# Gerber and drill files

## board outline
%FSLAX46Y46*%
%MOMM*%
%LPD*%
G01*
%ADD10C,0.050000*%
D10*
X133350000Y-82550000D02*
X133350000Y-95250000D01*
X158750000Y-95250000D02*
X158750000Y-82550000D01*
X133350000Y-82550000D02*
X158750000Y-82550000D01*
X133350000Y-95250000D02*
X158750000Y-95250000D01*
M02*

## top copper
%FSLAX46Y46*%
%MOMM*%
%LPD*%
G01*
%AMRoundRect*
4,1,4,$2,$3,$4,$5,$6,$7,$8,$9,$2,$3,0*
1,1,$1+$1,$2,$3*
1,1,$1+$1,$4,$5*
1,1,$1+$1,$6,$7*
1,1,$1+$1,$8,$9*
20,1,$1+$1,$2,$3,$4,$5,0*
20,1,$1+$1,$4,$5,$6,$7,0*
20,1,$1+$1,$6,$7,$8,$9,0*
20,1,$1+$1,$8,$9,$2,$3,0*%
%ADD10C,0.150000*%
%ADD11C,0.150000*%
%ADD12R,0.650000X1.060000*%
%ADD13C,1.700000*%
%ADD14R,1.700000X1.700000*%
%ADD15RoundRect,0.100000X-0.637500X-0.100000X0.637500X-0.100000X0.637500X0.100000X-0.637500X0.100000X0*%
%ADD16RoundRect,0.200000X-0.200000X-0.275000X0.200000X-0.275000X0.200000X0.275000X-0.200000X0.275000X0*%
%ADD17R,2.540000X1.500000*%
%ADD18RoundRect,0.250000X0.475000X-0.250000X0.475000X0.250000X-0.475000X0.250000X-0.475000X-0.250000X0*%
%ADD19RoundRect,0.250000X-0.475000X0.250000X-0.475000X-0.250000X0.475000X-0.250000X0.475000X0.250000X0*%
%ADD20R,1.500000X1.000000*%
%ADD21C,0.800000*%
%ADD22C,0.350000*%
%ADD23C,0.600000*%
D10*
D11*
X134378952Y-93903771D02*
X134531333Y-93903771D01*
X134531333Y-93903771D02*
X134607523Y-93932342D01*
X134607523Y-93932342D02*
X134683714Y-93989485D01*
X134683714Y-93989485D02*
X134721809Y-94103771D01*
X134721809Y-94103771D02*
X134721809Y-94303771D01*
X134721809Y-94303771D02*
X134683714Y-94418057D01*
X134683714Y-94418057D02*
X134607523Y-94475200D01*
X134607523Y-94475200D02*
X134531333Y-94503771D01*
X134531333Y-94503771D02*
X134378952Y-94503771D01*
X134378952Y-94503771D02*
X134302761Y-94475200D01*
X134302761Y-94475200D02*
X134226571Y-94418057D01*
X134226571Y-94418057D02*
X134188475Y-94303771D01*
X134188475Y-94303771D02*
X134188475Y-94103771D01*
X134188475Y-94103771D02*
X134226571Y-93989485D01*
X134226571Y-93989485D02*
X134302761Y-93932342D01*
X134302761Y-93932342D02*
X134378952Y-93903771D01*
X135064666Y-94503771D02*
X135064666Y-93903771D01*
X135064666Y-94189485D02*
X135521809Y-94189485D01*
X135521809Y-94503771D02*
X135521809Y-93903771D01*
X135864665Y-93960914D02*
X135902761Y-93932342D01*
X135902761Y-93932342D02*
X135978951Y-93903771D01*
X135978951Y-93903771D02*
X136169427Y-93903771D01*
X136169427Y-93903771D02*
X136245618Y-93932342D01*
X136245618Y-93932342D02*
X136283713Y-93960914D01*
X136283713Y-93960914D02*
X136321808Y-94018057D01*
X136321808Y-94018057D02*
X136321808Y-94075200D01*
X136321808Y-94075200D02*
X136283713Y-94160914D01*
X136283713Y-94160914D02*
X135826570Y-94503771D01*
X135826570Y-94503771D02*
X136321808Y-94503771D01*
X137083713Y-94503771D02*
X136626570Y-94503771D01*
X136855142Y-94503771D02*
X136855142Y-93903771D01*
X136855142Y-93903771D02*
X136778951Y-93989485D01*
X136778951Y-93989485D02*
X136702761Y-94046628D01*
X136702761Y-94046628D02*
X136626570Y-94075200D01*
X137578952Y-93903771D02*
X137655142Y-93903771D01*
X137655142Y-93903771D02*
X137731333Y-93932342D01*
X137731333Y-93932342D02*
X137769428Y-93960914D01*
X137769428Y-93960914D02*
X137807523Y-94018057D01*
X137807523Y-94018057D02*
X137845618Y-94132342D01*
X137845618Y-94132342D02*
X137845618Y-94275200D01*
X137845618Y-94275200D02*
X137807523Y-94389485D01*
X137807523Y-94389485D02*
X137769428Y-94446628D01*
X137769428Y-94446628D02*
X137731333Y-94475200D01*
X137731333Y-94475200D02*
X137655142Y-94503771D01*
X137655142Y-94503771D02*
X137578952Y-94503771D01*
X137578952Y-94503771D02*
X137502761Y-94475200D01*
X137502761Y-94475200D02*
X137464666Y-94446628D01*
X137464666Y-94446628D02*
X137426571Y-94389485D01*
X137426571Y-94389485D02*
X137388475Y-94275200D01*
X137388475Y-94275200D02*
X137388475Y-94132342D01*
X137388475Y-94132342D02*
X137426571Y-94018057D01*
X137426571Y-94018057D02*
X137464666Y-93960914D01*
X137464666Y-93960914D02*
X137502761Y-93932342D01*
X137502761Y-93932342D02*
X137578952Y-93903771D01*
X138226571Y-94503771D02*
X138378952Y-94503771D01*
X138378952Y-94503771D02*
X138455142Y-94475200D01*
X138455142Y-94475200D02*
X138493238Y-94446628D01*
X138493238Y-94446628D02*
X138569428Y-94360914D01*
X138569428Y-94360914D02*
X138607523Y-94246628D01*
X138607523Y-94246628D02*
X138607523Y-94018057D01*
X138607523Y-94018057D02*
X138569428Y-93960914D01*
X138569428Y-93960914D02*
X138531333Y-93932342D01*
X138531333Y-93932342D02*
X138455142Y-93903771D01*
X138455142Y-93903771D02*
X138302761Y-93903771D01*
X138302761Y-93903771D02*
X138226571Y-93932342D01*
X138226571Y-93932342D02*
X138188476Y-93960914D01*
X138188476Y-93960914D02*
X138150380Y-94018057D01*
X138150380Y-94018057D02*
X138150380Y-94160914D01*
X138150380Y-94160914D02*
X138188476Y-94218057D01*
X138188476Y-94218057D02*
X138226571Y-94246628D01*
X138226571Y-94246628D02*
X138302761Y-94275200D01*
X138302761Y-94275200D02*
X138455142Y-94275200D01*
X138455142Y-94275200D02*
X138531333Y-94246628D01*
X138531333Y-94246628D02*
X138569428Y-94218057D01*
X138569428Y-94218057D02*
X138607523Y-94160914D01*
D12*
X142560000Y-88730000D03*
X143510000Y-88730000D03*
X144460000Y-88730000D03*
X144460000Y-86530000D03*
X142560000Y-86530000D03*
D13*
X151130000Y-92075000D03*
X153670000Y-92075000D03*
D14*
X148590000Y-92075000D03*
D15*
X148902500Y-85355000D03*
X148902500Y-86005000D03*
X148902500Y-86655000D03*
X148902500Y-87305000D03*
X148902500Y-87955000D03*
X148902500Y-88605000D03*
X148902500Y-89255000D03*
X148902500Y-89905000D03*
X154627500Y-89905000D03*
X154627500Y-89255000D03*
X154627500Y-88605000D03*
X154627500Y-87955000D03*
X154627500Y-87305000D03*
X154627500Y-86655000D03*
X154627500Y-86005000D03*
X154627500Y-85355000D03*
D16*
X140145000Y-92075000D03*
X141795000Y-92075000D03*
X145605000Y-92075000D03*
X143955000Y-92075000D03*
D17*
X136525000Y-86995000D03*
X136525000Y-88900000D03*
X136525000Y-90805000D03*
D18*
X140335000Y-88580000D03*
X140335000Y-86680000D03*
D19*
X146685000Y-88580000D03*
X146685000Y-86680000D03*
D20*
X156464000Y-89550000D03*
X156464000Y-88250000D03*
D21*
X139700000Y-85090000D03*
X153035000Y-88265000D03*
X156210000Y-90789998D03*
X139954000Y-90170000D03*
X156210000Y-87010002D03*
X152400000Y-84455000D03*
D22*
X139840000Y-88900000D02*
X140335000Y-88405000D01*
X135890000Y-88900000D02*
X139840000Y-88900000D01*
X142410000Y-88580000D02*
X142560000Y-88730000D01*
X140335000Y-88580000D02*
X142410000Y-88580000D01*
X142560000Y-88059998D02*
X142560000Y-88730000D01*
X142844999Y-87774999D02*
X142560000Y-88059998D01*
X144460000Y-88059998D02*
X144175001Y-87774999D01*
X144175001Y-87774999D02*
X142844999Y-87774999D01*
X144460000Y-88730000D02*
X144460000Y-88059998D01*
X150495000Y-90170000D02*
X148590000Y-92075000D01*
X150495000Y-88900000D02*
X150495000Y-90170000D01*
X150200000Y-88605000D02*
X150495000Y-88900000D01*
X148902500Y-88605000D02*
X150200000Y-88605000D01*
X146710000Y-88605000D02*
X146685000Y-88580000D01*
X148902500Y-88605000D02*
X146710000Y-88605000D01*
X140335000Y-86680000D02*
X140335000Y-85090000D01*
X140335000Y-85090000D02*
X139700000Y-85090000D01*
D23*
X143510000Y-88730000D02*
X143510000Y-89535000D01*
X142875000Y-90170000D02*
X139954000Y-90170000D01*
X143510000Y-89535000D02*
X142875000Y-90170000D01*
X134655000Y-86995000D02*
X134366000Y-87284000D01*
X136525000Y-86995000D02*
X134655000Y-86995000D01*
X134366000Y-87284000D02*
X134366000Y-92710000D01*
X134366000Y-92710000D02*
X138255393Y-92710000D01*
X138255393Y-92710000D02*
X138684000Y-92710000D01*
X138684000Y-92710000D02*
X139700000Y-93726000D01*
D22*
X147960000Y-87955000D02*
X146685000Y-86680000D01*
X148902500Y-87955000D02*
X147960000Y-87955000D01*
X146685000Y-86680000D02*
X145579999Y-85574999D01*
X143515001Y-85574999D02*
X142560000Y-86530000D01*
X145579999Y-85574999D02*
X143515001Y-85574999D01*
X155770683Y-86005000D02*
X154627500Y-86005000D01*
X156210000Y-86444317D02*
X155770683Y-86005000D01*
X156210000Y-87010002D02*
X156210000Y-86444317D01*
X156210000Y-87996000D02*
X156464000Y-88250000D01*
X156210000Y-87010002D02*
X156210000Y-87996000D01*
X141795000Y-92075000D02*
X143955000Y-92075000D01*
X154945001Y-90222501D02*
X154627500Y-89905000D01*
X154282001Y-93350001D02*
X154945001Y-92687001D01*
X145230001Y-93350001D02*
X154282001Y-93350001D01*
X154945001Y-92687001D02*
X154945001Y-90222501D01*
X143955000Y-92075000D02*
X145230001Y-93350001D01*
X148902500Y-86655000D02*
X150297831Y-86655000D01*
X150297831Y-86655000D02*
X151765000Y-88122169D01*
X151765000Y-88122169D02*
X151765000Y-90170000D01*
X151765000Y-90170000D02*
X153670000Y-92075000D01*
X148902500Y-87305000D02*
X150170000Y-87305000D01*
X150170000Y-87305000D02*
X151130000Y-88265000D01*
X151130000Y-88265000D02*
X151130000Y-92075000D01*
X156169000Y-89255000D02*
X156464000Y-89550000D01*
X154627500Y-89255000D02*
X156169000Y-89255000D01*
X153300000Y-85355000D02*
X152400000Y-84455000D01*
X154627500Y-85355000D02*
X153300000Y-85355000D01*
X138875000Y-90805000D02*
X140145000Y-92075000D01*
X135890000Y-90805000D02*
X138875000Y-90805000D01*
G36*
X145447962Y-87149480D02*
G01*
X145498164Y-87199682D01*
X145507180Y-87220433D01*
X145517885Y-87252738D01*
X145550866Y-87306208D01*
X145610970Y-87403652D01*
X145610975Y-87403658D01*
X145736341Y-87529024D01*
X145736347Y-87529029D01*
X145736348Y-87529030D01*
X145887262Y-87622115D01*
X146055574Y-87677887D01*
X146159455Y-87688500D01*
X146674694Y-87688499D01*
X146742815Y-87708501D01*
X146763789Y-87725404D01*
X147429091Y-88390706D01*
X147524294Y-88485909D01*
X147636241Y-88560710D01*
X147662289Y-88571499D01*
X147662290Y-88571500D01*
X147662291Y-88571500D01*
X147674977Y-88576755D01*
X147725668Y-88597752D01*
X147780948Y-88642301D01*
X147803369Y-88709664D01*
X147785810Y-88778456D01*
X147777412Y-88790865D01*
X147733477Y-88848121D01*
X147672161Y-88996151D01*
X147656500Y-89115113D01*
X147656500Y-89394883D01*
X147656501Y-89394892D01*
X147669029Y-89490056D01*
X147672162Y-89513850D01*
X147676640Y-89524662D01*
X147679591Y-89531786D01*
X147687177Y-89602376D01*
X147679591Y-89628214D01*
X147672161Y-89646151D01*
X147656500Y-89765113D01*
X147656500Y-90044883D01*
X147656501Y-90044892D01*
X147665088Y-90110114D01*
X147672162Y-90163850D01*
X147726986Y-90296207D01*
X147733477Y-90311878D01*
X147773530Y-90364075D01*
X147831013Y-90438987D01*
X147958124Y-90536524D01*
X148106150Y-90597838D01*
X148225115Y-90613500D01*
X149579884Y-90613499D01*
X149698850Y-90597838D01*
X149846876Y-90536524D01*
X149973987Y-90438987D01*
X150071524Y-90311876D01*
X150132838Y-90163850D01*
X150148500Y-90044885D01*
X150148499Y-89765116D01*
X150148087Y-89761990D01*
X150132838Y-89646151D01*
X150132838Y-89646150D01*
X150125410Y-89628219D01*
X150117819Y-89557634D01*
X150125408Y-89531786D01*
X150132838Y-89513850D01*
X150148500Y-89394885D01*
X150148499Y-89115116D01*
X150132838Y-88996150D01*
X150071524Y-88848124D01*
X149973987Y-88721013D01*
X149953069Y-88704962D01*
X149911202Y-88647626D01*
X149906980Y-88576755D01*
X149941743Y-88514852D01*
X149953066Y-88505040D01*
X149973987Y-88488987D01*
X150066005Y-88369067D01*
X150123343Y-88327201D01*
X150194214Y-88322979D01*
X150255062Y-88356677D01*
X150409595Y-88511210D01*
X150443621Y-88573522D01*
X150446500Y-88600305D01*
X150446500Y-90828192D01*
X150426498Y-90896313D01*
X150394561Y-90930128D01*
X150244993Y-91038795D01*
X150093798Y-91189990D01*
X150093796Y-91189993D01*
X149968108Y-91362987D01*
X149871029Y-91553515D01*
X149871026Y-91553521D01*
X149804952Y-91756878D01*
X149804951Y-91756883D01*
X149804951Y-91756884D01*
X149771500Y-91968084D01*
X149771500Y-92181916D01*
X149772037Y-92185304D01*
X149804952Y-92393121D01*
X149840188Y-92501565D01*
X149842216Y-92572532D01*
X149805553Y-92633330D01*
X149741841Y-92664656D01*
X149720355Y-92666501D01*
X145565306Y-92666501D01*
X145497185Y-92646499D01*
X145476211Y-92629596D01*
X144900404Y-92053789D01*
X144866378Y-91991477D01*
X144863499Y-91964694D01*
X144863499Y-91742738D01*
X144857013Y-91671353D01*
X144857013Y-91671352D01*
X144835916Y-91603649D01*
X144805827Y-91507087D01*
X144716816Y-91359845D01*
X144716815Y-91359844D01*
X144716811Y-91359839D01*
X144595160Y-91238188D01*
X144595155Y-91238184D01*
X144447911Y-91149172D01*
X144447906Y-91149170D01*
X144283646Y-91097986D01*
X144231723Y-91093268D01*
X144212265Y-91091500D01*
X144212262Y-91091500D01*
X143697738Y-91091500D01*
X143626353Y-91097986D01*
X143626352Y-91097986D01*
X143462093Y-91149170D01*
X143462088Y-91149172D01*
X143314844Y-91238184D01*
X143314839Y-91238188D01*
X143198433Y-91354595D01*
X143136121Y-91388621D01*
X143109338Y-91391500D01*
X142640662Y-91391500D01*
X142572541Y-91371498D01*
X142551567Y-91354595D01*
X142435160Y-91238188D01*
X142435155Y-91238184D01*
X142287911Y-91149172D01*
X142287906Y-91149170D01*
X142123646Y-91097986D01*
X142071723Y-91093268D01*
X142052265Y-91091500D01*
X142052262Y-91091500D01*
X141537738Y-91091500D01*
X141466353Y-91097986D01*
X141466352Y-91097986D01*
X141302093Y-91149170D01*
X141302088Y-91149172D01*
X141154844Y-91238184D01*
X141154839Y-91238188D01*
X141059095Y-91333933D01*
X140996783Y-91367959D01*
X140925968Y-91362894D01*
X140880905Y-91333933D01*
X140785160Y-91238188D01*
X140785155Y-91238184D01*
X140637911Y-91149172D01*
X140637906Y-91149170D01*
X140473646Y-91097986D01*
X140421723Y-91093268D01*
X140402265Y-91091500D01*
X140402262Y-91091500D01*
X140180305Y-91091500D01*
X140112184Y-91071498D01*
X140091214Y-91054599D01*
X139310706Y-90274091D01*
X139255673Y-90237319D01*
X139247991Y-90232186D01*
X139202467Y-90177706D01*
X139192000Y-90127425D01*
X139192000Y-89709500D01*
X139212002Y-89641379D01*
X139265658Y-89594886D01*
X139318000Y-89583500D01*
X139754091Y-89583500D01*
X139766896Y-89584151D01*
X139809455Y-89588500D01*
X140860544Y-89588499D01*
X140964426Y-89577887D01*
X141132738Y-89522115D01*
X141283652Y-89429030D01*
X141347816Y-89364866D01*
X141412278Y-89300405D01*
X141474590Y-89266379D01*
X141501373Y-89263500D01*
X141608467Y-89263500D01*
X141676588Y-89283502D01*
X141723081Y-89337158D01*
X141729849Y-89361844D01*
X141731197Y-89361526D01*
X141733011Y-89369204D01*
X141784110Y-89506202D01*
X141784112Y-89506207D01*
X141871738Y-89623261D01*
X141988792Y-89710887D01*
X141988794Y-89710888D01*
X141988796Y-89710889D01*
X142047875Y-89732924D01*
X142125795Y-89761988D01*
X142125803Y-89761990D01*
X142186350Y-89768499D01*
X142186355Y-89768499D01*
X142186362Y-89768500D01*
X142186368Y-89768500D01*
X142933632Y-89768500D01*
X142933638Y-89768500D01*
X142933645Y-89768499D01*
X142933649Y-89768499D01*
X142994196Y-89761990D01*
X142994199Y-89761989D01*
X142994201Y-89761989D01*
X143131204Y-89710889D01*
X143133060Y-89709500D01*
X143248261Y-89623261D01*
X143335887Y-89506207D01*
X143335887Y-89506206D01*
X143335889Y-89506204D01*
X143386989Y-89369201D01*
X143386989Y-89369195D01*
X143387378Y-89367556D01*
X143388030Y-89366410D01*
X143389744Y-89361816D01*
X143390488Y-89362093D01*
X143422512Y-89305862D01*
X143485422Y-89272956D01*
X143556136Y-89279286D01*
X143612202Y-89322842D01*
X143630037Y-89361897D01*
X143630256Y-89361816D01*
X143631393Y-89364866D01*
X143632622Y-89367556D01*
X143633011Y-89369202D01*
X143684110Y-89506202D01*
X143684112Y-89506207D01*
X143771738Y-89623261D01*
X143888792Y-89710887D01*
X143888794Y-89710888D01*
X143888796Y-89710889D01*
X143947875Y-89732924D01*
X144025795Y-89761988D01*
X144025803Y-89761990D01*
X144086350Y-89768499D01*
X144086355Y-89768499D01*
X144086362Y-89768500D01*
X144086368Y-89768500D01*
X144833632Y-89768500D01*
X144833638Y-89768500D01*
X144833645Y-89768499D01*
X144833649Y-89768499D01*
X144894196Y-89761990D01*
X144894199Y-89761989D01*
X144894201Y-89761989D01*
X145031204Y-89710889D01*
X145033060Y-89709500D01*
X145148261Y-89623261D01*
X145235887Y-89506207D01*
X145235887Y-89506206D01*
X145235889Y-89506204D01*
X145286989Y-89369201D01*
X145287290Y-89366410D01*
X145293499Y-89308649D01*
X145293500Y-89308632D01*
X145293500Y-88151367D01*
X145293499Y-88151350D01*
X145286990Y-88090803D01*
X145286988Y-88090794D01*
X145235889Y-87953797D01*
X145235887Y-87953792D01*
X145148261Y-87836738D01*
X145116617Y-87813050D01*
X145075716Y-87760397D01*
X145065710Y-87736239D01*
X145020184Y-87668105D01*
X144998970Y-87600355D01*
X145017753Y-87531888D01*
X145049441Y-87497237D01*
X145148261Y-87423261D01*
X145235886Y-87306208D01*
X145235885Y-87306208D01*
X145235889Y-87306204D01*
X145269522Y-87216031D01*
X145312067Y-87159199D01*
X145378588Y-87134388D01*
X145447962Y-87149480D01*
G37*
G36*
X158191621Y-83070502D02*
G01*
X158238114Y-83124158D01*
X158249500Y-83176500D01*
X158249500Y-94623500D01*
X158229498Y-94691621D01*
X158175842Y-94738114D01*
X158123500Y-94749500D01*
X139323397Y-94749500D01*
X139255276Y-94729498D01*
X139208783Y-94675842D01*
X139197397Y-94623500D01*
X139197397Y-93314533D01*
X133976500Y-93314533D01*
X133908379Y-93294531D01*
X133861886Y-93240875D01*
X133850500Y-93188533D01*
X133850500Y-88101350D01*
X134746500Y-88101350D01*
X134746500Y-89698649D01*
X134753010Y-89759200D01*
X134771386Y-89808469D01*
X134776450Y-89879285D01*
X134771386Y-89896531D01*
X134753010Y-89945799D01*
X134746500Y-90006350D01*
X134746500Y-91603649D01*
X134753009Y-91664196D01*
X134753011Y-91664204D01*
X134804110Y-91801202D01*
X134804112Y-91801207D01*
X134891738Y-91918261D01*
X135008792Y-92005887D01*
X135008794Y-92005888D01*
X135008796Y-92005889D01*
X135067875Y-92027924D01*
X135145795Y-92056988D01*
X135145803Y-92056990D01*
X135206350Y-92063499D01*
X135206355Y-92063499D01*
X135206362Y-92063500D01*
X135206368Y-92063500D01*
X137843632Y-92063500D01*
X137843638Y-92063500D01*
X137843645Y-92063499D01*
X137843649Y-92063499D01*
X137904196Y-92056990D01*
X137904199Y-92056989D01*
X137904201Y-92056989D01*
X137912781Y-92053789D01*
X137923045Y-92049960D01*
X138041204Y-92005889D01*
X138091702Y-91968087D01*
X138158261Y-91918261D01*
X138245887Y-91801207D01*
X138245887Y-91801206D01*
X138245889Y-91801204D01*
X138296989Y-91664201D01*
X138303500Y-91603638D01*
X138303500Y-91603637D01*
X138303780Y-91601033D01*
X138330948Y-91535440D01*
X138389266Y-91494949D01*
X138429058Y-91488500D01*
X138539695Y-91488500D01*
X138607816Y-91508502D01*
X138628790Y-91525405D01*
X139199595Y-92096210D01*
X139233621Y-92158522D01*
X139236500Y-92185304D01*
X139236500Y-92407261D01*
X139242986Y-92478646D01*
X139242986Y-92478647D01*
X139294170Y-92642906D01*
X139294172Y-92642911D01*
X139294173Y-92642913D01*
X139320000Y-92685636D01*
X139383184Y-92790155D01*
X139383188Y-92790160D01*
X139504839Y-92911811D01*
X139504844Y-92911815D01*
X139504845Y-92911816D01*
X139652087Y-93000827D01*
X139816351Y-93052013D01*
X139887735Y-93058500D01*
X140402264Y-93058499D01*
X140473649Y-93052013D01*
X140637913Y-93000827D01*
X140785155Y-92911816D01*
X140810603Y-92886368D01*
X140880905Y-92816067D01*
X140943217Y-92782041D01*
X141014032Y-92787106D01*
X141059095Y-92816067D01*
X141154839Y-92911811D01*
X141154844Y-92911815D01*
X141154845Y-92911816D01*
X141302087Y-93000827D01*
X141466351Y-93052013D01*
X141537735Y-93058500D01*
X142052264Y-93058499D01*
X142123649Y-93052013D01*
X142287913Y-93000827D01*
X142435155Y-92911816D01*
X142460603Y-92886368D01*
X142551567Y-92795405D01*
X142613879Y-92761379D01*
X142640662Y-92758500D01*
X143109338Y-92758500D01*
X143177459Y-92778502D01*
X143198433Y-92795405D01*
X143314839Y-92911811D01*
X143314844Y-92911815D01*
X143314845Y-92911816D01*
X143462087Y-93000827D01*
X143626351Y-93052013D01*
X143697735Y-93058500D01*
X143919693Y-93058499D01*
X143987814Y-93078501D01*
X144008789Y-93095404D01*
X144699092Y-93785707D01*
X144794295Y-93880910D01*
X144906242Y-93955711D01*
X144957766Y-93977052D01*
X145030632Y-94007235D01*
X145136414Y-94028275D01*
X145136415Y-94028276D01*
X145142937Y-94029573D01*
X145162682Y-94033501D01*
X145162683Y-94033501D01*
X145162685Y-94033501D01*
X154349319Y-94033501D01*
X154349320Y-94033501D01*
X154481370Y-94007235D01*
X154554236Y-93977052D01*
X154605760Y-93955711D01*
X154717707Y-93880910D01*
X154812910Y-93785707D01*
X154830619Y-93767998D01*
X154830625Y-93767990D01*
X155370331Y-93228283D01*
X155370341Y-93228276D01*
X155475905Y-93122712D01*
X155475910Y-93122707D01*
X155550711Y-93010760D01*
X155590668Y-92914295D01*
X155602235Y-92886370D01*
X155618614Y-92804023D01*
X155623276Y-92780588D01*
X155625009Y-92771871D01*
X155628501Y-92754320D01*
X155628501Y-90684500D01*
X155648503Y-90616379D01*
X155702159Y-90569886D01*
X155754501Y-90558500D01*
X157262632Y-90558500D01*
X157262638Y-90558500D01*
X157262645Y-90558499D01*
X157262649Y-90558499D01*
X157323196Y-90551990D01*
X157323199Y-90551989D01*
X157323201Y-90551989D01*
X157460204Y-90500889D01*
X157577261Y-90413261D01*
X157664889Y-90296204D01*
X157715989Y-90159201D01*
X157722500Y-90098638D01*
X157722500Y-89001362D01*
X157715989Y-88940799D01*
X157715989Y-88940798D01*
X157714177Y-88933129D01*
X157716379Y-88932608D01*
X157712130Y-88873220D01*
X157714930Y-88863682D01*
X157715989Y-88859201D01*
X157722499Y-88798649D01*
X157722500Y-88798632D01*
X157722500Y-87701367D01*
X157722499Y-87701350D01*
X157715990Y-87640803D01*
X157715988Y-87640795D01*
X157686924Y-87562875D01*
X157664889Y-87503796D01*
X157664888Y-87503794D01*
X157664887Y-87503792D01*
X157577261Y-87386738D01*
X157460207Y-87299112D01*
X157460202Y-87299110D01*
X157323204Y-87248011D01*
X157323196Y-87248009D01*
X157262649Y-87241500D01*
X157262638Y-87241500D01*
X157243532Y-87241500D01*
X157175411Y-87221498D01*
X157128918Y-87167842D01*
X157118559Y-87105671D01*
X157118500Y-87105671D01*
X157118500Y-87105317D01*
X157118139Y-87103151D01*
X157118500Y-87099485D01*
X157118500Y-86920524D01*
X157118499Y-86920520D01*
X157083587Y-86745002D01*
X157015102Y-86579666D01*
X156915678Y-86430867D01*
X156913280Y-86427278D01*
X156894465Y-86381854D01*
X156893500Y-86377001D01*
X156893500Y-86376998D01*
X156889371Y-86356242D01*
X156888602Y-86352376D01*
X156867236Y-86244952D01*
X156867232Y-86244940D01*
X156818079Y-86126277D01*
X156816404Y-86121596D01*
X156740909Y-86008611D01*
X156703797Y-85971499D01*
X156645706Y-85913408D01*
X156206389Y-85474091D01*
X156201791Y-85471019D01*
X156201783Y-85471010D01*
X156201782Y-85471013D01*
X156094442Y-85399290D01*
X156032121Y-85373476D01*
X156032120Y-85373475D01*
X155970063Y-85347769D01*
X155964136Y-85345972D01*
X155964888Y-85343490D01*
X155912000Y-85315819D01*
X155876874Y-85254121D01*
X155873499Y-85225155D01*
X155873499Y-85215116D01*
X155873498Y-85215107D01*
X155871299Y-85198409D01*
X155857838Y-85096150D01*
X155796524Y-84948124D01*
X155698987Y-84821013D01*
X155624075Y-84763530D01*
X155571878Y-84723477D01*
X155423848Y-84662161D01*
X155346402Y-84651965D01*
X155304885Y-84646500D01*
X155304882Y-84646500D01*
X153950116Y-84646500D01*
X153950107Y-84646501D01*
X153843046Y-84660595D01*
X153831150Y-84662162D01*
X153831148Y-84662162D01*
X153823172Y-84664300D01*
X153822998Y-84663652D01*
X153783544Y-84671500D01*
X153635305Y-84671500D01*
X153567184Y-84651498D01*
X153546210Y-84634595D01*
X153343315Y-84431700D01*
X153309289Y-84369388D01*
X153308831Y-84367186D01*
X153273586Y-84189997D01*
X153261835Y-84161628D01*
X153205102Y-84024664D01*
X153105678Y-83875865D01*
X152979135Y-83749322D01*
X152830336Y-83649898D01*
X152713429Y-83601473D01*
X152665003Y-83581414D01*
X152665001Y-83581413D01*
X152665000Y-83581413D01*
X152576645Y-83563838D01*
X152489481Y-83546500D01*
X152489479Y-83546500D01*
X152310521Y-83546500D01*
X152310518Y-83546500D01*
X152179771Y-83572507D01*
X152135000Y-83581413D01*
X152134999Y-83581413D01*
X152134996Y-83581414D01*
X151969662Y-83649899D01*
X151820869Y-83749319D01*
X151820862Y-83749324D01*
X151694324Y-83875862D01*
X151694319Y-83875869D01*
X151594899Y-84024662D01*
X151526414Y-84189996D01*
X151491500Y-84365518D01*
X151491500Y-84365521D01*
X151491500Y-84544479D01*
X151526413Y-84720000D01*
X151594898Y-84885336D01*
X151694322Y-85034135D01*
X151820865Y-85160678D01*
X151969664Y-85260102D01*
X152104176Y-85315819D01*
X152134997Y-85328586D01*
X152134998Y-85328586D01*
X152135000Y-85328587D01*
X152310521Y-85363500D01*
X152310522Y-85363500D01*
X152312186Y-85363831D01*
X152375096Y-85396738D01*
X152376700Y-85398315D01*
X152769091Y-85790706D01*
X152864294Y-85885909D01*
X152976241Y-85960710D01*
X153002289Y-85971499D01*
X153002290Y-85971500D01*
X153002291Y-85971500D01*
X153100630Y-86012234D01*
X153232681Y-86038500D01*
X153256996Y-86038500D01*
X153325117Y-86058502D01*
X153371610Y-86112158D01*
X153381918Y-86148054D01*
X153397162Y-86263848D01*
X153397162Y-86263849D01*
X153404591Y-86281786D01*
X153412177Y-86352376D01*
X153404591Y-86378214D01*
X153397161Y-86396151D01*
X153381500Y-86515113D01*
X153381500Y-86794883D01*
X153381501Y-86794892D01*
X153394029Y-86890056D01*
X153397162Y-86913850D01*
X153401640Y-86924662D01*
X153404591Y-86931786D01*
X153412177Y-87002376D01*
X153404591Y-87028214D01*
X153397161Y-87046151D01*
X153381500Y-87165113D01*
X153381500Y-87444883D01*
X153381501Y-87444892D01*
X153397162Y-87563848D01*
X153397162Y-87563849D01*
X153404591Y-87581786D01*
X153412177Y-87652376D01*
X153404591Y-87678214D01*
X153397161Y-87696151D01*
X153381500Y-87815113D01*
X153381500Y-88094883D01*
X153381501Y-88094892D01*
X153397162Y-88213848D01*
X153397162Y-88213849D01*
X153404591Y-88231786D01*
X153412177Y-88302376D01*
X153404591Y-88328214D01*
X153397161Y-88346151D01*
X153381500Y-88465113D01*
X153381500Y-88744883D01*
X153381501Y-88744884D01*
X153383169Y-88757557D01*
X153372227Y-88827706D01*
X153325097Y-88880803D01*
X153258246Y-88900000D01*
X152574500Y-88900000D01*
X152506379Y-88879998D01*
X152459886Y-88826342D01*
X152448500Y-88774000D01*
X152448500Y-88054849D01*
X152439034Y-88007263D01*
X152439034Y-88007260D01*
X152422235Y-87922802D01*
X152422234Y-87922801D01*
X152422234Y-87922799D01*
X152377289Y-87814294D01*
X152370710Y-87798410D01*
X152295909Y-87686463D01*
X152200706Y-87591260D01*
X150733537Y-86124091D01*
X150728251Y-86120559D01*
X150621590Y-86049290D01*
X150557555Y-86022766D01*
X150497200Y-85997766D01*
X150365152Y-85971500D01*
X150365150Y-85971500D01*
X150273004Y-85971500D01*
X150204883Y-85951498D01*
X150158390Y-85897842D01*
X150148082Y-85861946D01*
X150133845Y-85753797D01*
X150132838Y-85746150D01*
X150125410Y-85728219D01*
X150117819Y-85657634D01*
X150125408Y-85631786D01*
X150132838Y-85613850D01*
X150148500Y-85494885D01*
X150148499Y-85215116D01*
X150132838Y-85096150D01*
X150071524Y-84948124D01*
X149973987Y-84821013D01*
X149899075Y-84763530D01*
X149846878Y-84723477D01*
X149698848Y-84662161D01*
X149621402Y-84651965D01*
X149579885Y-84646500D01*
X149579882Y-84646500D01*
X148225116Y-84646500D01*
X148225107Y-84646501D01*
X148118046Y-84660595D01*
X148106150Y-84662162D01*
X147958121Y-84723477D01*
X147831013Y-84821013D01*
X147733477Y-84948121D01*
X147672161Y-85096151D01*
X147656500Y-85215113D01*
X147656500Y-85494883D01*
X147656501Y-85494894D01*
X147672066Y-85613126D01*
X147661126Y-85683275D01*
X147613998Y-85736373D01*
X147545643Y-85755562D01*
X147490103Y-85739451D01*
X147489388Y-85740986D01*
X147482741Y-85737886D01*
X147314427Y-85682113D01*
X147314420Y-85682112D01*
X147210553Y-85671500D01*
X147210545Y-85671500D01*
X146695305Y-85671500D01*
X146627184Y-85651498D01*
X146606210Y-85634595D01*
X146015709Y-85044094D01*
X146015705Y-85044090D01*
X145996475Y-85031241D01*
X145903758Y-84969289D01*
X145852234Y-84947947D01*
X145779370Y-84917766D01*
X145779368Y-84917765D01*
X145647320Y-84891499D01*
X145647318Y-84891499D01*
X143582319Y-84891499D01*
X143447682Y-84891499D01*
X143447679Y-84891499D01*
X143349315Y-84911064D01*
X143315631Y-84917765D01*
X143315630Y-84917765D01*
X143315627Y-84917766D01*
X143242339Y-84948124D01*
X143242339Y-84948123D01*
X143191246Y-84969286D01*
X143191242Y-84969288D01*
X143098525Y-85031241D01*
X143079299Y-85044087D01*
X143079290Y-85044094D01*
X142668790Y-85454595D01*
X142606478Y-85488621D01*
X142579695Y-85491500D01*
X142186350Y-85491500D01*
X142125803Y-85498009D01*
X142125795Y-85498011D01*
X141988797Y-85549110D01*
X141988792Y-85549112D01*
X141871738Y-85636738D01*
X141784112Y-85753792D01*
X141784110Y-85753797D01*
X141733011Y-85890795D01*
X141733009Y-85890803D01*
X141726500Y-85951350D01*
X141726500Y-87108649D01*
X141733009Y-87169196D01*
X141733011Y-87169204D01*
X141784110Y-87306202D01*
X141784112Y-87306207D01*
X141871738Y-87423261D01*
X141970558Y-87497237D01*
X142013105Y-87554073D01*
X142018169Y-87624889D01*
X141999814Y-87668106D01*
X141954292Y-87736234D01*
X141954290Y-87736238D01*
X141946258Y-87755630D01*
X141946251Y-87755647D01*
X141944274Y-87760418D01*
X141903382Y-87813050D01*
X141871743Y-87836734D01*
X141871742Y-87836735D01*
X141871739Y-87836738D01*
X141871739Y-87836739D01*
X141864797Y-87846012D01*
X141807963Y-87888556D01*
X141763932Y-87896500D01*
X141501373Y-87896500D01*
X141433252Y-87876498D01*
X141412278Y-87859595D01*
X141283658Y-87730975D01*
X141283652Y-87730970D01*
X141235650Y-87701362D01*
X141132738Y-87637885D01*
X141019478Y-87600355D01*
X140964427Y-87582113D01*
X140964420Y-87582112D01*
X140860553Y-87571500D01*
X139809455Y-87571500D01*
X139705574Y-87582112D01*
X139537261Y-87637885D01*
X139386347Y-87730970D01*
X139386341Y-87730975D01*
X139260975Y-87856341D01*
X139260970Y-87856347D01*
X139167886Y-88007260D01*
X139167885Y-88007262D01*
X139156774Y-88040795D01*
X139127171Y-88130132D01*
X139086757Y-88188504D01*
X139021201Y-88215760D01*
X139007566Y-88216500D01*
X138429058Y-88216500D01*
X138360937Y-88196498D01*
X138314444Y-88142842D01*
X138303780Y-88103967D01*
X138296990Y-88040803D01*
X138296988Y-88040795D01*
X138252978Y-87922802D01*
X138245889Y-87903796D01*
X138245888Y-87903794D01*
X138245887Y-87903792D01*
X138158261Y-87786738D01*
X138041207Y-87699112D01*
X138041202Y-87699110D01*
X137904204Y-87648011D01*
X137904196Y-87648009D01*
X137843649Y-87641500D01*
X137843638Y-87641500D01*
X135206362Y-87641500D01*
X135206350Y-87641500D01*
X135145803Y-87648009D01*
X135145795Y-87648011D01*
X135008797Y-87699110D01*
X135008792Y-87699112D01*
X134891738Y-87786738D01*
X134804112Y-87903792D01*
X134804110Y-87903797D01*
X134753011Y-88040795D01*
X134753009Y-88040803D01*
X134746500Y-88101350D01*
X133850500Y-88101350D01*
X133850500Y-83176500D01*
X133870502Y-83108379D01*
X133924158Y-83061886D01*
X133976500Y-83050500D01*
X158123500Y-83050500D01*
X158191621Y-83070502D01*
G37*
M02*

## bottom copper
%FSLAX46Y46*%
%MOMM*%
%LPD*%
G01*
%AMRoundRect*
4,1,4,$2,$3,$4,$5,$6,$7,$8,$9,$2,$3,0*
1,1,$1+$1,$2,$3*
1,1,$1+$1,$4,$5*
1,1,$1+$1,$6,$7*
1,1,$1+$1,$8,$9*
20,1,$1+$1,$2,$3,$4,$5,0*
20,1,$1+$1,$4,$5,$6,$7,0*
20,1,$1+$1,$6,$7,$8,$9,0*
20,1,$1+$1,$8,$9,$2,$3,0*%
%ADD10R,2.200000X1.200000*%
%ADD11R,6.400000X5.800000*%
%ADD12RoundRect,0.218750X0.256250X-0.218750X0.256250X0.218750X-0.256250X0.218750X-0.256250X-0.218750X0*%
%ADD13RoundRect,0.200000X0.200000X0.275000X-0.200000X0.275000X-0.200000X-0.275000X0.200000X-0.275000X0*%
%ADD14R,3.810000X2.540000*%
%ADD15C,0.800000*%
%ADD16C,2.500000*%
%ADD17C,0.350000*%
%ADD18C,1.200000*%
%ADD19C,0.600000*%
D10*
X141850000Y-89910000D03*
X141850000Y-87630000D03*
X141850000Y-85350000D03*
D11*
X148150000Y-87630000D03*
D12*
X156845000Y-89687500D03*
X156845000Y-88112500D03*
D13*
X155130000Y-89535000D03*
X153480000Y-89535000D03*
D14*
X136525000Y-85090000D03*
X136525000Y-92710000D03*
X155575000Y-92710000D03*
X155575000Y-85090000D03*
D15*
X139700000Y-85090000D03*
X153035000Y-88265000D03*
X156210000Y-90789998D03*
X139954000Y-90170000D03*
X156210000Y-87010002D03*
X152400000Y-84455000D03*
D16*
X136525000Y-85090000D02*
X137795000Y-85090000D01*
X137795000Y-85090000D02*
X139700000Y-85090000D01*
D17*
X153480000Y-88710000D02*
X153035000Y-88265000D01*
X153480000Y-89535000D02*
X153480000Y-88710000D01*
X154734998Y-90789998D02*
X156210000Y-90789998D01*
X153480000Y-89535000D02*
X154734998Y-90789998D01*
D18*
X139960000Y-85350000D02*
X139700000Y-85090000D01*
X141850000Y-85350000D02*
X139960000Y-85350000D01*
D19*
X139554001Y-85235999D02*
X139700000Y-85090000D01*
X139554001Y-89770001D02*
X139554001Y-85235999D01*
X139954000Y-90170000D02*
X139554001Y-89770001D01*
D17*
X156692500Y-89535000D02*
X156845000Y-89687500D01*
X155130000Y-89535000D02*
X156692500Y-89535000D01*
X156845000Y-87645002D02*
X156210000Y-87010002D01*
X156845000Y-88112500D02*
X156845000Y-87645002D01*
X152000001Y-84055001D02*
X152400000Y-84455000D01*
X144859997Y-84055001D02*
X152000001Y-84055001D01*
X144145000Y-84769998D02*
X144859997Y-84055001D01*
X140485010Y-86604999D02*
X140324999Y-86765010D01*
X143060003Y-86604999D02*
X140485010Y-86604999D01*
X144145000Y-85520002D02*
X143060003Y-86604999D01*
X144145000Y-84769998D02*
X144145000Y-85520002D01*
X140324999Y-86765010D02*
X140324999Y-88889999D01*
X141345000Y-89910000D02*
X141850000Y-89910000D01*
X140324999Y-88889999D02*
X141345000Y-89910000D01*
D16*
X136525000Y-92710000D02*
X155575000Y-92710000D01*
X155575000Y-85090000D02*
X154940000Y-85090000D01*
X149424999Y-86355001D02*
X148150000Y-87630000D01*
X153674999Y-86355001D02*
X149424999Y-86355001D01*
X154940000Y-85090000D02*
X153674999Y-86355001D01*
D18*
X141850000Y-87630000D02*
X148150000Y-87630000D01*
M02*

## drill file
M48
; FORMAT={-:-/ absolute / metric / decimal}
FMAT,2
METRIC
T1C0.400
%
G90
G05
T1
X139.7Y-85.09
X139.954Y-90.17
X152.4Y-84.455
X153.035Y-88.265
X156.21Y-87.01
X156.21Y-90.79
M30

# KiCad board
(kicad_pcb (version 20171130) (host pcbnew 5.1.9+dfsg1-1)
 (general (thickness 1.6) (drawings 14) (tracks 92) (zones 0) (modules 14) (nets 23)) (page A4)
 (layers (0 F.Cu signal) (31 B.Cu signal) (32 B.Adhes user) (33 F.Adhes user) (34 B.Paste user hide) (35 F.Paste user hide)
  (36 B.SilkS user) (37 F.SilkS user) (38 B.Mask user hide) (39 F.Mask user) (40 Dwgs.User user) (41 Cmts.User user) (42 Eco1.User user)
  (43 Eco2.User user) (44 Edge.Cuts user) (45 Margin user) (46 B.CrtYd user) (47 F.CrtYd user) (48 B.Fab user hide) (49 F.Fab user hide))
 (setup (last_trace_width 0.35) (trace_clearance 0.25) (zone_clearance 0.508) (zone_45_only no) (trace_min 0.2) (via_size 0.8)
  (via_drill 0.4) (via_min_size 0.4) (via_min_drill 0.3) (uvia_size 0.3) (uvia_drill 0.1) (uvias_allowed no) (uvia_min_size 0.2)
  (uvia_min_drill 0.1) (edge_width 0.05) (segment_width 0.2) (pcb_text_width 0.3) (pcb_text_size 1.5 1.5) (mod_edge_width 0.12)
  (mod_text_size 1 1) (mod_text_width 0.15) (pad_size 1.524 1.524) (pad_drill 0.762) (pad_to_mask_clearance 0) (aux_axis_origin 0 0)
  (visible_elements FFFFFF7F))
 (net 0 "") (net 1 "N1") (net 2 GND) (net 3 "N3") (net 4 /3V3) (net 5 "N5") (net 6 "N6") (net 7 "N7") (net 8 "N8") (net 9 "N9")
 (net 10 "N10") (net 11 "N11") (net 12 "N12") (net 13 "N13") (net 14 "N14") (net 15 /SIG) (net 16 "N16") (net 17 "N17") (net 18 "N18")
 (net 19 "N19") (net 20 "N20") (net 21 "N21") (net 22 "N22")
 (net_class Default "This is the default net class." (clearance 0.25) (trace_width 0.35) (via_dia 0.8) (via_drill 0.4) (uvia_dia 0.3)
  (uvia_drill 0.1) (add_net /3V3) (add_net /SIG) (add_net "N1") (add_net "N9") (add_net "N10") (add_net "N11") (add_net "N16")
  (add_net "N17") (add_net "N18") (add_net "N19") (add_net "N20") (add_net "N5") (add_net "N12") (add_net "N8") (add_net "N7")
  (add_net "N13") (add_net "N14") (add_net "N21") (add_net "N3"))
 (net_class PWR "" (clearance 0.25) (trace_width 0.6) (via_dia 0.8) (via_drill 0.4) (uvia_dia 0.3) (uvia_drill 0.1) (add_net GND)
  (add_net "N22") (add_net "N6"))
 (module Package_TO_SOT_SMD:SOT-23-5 (layer F.Cu) (at 143.51 87.63 90)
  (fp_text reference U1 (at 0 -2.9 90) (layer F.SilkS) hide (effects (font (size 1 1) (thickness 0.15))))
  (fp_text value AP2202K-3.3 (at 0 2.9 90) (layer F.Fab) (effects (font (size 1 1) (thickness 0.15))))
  (pad 1 smd rect (at -1.1 -0.95 90) (size 1.06 0.65) (layers F.Cu F.Paste F.Mask) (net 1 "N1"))
  (pad 2 smd rect (at -1.1 0 90) (size 1.06 0.65) (layers F.Cu F.Paste F.Mask) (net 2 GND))
  (pad 3 smd rect (at -1.1 0.95 90) (size 1.06 0.65) (layers F.Cu F.Paste F.Mask) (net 1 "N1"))
  (pad 4 smd rect (at 1.1 0.95 90) (size 1.06 0.65) (layers F.Cu F.Paste F.Mask) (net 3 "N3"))
  (pad 5 smd rect (at 1.1 -0.95 90) (size 1.06 0.65) (layers F.Cu F.Paste F.Mask) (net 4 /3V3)))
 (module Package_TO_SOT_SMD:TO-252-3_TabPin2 (layer B.Cu) (at 146.05 87.63)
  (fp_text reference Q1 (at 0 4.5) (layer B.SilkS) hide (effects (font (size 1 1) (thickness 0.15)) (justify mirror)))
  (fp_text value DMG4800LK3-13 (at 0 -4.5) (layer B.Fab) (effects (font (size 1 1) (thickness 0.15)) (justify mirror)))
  (pad 1 smd rect (at -4.2 2.28) (size 2.2 1.2) (layers B.Cu B.Paste B.Mask) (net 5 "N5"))
  (pad 2 smd rect (at -4.2 0) (size 2.2 1.2) (layers B.Cu B.Paste B.Mask) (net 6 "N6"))
  (pad 3 smd rect (at -4.2 -2.28) (size 2.2 1.2) (layers B.Cu B.Paste B.Mask) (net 2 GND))
  (pad 2 smd rect (at 2.1 0) (size 6.4 5.8) (layers B.Cu B.Mask) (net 6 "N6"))
  (pad "" smd rect (at 3.775 -1.525) (size 3.05 2.75) (layers B.Paste))
  (pad "" smd rect (at 0.425 1.525) (size 3.05 2.75) (layers B.Paste))
  (pad "" smd rect (at 3.775 1.525) (size 3.05 2.75) (layers B.Paste))
  (pad "" smd rect (at 0.425 -1.525) (size 3.05 2.75) (layers B.Paste)))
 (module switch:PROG (layer F.Cu) (at 151.13 92.075 90)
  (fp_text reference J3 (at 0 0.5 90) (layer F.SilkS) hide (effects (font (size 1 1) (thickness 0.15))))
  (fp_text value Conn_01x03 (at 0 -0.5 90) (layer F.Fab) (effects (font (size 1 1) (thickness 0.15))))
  (pad 2 smd circle (at 0 0 90) (size 1.7 1.7) (layers F.Cu F.Paste F.Mask) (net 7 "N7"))
  (pad 3 smd circle (at 0 2.54 90) (size 1.7 1.7) (layers F.Cu F.Paste F.Mask) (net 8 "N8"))
  (pad 1 smd rect (at 0 -2.54 90) (size 1.7 1.7) (layers F.Cu F.Paste F.Mask) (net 2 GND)))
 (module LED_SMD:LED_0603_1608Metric (layer B.Cu) (at 156.845 88.9 90)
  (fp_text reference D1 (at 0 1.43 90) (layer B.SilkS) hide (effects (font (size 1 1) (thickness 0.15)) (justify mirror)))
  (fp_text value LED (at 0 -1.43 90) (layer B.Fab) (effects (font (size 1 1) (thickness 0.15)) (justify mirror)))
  (pad 1 smd roundrect (at -0.7875 0 90) (size 0.875 0.95) (layers B.Cu B.Paste B.Mask) (roundrect_rratio 0.25) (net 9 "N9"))
  (pad 2 smd roundrect (at 0.7875 0 90) (size 0.875 0.95) (layers B.Cu B.Paste B.Mask) (roundrect_rratio 0.25) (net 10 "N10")))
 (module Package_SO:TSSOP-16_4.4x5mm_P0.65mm (layer F.Cu) (at 151.765 87.63)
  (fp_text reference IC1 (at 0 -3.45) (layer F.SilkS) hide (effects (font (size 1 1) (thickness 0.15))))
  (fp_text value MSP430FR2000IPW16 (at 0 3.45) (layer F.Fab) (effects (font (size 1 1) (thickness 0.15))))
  (pad 1 smd roundrect (at -2.8625 -2.275) (size 1.475 0.4) (layers F.Cu F.Paste F.Mask) (roundrect_rratio 0.25) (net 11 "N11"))
  (pad 2 smd roundrect (at -2.8625 -1.625) (size 1.475 0.4) (layers F.Cu F.Paste F.Mask) (roundrect_rratio 0.25) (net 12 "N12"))
  (pad 3 smd roundrect (at -2.8625 -0.975) (size 1.475 0.4) (layers F.Cu F.Paste F.Mask) (roundrect_rratio 0.25) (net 8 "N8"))
  (pad 4 smd roundrect (at -2.8625 -0.325) (size 1.475 0.4) (layers F.Cu F.Paste F.Mask) (roundrect_rratio 0.25) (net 7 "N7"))
  (pad 5 smd roundrect (at -2.8625 0.325) (size 1.475 0.4) (layers F.Cu F.Paste F.Mask) (roundrect_rratio 0.25) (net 4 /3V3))
  (pad 6 smd roundrect (at -2.8625 0.975) (size 1.475 0.4) (layers F.Cu F.Paste F.Mask) (roundrect_rratio 0.25) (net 2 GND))
  (pad 7 smd roundrect (at -2.8625 1.625) (size 1.475 0.4) (layers F.Cu F.Paste F.Mask) (roundrect_rratio 0.25) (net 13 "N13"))
  (pad 8 smd roundrect (at -2.8625 2.275) (size 1.475 0.4) (layers F.Cu F.Paste F.Mask) (roundrect_rratio 0.25) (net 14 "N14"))
  (pad 9 smd roundrect (at 2.8625 2.275) (size 1.475 0.4) (layers F.Cu F.Paste F.Mask) (roundrect_rratio 0.25) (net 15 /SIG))
  (pad 10 smd roundrect (at 2.8625 1.625) (size 1.475 0.4) (layers F.Cu F.Paste F.Mask) (roundrect_rratio 0.25) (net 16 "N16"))
  (pad 11 smd roundrect (at 2.8625 0.975) (size 1.475 0.4) (layers F.Cu F.Paste F.Mask) (roundrect_rratio 0.25) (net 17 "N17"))
  (pad 12 smd roundrect (at 2.8625 0.325) (size 1.475 0.4) (layers F.Cu F.Paste F.Mask) (roundrect_rratio 0.25) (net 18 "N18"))
  (pad 13 smd roundrect (at 2.8625 -0.325) (size 1.475 0.4) (layers F.Cu F.Paste F.Mask) (roundrect_rratio 0.25) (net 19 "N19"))
  (pad 14 smd roundrect (at 2.8625 -0.975) (size 1.475 0.4) (layers F.Cu F.Paste F.Mask) (roundrect_rratio 0.25) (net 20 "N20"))
  (pad 15 smd roundrect (at 2.8625 -1.625) (size 1.475 0.4) (layers F.Cu F.Paste F.Mask) (roundrect_rratio 0.25) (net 10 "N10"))
  (pad 16 smd roundrect (at 2.8625 -2.275) (size 1.475 0.4) (layers F.Cu F.Paste F.Mask) (roundrect_rratio 0.25) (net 5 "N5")))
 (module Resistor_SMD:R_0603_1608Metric (layer F.Cu) (at 140.97 92.075)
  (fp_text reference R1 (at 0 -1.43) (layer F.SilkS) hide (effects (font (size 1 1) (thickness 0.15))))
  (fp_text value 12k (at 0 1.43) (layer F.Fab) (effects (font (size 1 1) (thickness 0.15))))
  (pad 1 smd roundrect (at -0.825 0) (size 0.8 0.95) (layers F.Cu F.Paste F.Mask) (roundrect_rratio 0.25) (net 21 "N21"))
  (pad 2 smd roundrect (at 0.825 0) (size 0.8 0.95) (layers F.Cu F.Paste F.Mask) (roundrect_rratio 0.25) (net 15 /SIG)))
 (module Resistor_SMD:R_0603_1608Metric (layer F.Cu) (at 144.78 92.075)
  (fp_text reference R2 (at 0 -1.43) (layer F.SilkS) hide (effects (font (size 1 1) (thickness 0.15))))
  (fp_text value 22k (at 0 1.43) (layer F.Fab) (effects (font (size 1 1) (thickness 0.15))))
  (pad 2 smd roundrect (at 0.825 0) (size 0.8 0.95) (layers F.Cu F.Paste F.Mask) (roundrect_rratio 0.25) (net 2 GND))
  (pad 1 smd roundrect (at -0.825 0) (size 0.8 0.95) (layers F.Cu F.Paste F.Mask) (roundrect_rratio 0.25) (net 15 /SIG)))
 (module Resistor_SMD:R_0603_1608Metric (layer B.Cu) (at 154.305 89.535 180)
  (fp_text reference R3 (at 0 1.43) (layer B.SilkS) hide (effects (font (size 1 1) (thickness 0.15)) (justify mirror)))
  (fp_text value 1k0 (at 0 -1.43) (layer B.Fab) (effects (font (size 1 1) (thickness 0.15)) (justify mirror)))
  (pad 1 smd roundrect (at -0.825 0 180) (size 0.8 0.95) (layers B.Cu B.Paste B.Mask) (roundrect_rratio 0.25) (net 9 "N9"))
  (pad 2 smd roundrect (at 0.825 0 180) (size 0.8 0.95) (layers B.Cu B.Paste B.Mask) (roundrect_rratio 0.25) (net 2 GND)))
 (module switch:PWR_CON (layer B.Cu) (at 136.525 88.9 180)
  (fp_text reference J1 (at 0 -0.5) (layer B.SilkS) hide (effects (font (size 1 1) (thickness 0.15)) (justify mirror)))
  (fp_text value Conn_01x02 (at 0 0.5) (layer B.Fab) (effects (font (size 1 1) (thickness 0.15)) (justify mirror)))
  (pad 1 smd rect (at 0 3.81 180) (size 3.81 2.54) (layers B.Cu B.Paste B.Mask) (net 2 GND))
  (pad 2 smd rect (at 0 -3.81 180) (size 3.81 2.54) (layers B.Cu B.Paste B.Mask) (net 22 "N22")))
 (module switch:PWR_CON (layer B.Cu) (at 155.575 88.9 180)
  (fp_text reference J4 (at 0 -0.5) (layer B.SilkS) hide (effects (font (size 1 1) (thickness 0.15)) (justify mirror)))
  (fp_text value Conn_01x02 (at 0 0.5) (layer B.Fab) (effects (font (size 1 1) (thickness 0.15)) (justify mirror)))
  (pad 2 smd rect (at 0 -3.81 180) (size 3.81 2.54) (layers B.Cu B.Paste B.Mask) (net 22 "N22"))
  (pad 1 smd rect (at 0 3.81 180) (size 3.81 2.54) (layers B.Cu B.Paste B.Mask) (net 6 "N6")))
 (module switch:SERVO (layer F.Cu) (at 136.525 88.9)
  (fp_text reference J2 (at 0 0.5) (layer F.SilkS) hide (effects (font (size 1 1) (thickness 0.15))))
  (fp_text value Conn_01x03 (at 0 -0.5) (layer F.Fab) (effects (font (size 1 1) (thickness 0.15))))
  (pad 1 smd rect (at 0 -1.905) (size 2.54 1.5) (layers F.Cu F.Paste F.Mask) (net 2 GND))
  (pad 2 smd rect (at 0 0) (size 2.54 1.5) (layers F.Cu F.Paste F.Mask) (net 1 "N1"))
  (pad 3 smd rect (at 0 1.905) (size 2.54 1.5) (layers F.Cu F.Paste F.Mask) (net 21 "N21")))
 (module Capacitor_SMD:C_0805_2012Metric (layer F.Cu) (at 140.335 87.63 90)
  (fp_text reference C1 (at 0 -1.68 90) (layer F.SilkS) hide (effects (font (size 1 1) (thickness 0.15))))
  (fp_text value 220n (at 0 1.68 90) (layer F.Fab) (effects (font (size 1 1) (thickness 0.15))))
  (pad 1 smd roundrect (at -0.95 0 90) (size 1 1.45) (layers F.Cu F.Paste F.Mask) (roundrect_rratio 0.25) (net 1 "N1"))
  (pad 2 smd roundrect (at 0.95 0 90) (size 1 1.45) (layers F.Cu F.Paste F.Mask) (roundrect_rratio 0.25) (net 2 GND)))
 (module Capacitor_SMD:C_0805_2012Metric (layer F.Cu) (at 146.685 87.63 270)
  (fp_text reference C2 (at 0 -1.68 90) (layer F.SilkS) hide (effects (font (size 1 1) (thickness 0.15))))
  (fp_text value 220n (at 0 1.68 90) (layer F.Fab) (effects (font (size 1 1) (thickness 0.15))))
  (pad 2 smd roundrect (at 0.95 0 270) (size 1 1.45) (layers F.Cu F.Paste F.Mask) (roundrect_rratio 0.25) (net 2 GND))
  (pad 1 smd roundrect (at -0.95 0 270) (size 1 1.45) (layers F.Cu F.Paste F.Mask) (roundrect_rratio 0.25) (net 4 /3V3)))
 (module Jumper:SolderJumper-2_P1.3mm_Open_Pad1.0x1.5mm (layer F.Cu) (at 156.464 88.9 270)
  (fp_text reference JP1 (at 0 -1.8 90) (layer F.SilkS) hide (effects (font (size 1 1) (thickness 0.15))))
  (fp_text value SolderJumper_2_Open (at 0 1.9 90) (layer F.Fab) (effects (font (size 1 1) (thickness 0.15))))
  (pad 2 smd rect (at 0.65 0 270) (size 1 1.5) (layers F.Cu F.Mask) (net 16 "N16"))
  (pad 1 smd rect (at -0.65 0 270) (size 1 1.5) (layers F.Cu F.Mask) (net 10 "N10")))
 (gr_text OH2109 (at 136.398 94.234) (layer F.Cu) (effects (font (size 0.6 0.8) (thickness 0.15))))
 (gr_line (start 133.35 82.55) (end 133.35 95.25) (layer Edge.Cuts) (width 0.05))
 (gr_line (start 158.75 95.25) (end 158.75 82.55) (layer Edge.Cuts) (width 0.05))
 (gr_line (start 133.35 82.55) (end 158.75 82.55) (layer Edge.Cuts) (width 0.05))
 (gr_line (start 133.35 95.25) (end 158.75 95.25) (layer Edge.Cuts) (width 0.05))
 (segment (start 139.84 88.9) (end 140.335 88.405) (width 0.35) (layer F.Cu) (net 1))
 (segment (start 135.89 88.9) (end 139.84 88.9) (width 0.35) (layer F.Cu) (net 1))
 (segment (start 142.41 88.58) (end 142.56 88.73) (width 0.35) (layer F.Cu) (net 1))
 (segment (start 140.335 88.58) (end 142.41 88.58) (width 0.35) (layer F.Cu) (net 1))
 (segment (start 142.56 88.059998) (end 142.56 88.73) (width 0.35) (layer F.Cu) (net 1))
 (segment (start 142.844999 87.774999) (end 142.56 88.059998) (width 0.35) (layer F.Cu) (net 1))
 (segment (start 144.46 88.059998) (end 144.175001 87.774999) (width 0.35) (layer F.Cu) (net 1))
 (segment (start 144.175001 87.774999) (end 142.844999 87.774999) (width 0.35) (layer F.Cu) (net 1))
 (segment (start 144.46 88.73) (end 144.46 88.059998) (width 0.35) (layer F.Cu) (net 1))
 (segment (start 136.525 85.09) (end 137.795 85.09) (width 2.5) (layer B.Cu) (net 2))
 (segment (start 150.495 90.17) (end 148.59 92.075) (width 0.35) (layer F.Cu) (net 2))
 (segment (start 150.495 88.9) (end 150.495 90.17) (width 0.35) (layer F.Cu) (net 2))
 (segment (start 150.2 88.605) (end 150.495 88.9) (width 0.35) (layer F.Cu) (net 2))
 (segment (start 148.9025 88.605) (end 150.2 88.605) (width 0.35) (layer F.Cu) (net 2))
 (segment (start 146.71 88.605) (end 146.685 88.58) (width 0.35) (layer F.Cu) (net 2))
 (segment (start 148.9025 88.605) (end 146.71 88.605) (width 0.35) (layer F.Cu) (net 2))
 (segment (start 140.335 86.68) (end 140.335 85.09) (width 0.35) (layer F.Cu) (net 2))
 (via (at 139.7 85.09) (size 0.8) (drill 0.4) (layers F.Cu B.Cu) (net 2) (status 1000000))
 (segment (start 140.335 85.09) (end 139.7 85.09) (width 0.35) (layer F.Cu) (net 2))
 (segment (start 137.795 85.09) (end 139.7 85.09) (width 2.5) (layer B.Cu) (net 2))
 (via (at 153.035 88.265) (size 0.8) (drill 0.4) (layers F.Cu B.Cu) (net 2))
 (segment (start 153.48 88.71) (end 153.035 88.265) (width 0.35) (layer B.Cu) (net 2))
 (segment (start 153.48 89.535) (end 153.48 88.71) (width 0.35) (layer B.Cu) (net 2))
 (via (at 156.21 90.789998) (size 0.8) (drill 0.4) (layers F.Cu B.Cu) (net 2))
 (segment (start 154.734998 90.789998) (end 156.21 90.789998) (width 0.35) (layer B.Cu) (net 2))
 (segment (start 153.48 89.535) (end 154.734998 90.789998) (width 0.35) (layer B.Cu) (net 2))
 (segment (start 139.96 85.35) (end 139.7 85.09) (width 1.2) (layer B.Cu) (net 2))
 (segment (start 141.85 85.35) (end 139.96 85.35) (width 1.2) (layer B.Cu) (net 2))
 (via (at 139.954 90.17) (size 0.8) (drill 0.4) (layers F.Cu B.Cu) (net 2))
 (segment (start 139.554001 85.235999) (end 139.7 85.09) (width 0.6) (layer B.Cu) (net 2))
 (segment (start 139.554001 89.770001) (end 139.554001 85.235999) (width 0.6) (layer B.Cu) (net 2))
 (segment (start 139.954 90.17) (end 139.554001 89.770001) (width 0.6) (layer B.Cu) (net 2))
 (segment (start 143.51 88.73) (end 143.51 89.535) (width 0.6) (layer F.Cu) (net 2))
 (segment (start 142.875 90.17) (end 139.954 90.17) (width 0.6) (layer F.Cu) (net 2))
 (segment (start 143.51 89.535) (end 142.875 90.17) (width 0.6) (layer F.Cu) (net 2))
 (segment (start 134.655 86.995) (end 134.366 87.284) (width 0.6) (layer F.Cu) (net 2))
 (segment (start 136.525 86.995) (end 134.655 86.995) (width 0.6) (layer F.Cu) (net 2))
 (segment (start 134.366 87.284) (end 134.366 92.71) (width 0.6) (layer F.Cu) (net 2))
 (segment (start 134.366 92.71) (end 138.255393 92.71) (width 0.6) (layer F.Cu) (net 2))
 (segment (start 138.255393 92.71) (end 138.684 92.71) (width 0.6) (layer F.Cu) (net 2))
 (segment (start 138.684 92.71) (end 139.7 93.726) (width 0.6) (layer F.Cu) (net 2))
 (segment (start 147.96 87.955) (end 146.685 86.68) (width 0.35) (layer F.Cu) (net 4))
 (segment (start 148.9025 87.955) (end 147.96 87.955) (width 0.35) (layer F.Cu) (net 4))
 (segment (start 146.685 86.68) (end 145.579999 85.574999) (width 0.35) (layer F.Cu) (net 4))
 (segment (start 143.515001 85.574999) (end 142.56 86.53) (width 0.35) (layer F.Cu) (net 4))
 (segment (start 145.579999 85.574999) (end 143.515001 85.574999) (width 0.35) (layer F.Cu) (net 4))
 (segment (start 156.6925 89.535) (end 156.845 89.6875) (width 0.35) (layer B.Cu) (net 9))
 (segment (start 155.13 89.535) (end 156.6925 89.535) (width 0.35) (layer B.Cu) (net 9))
 (via (at 156.21 87.010002) (size 0.8) (drill 0.4) (layers F.Cu B.Cu) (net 10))
 (segment (start 156.845 87.645002) (end 156.21 87.010002) (width 0.35) (layer B.Cu) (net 10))
 (segment (start 156.845 88.1125) (end 156.845 87.645002) (width 0.35) (layer B.Cu) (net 10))
 (segment (start 155.770683 86.005) (end 154.6275 86.005) (width 0.35) (layer F.Cu) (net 10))
 (segment (start 156.21 86.444317) (end 155.770683 86.005) (width 0.35) (layer F.Cu) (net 10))
 (segment (start 156.21 87.010002) (end 156.21 86.444317) (width 0.35) (layer F.Cu) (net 10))
 (segment (start 156.21 87.996) (end 156.464 88.25) (width 0.35) (layer F.Cu) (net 10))
 (segment (start 156.21 87.010002) (end 156.21 87.996) (width 0.35) (layer F.Cu) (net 10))
 (segment (start 141.795 92.075) (end 143.955 92.075) (width 0.35) (layer F.Cu) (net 15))
 (segment (start 154.945001 90.222501) (end 154.6275 89.905) (width 0.35) (layer F.Cu) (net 15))
 (segment (start 154.282001 93.350001) (end 154.945001 92.687001) (width 0.35) (layer F.Cu) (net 15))
 (segment (start 145.230001 93.350001) (end 154.282001 93.350001) (width 0.35) (layer F.Cu) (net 15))
 (segment (start 154.945001 92.687001) (end 154.945001 90.222501) (width 0.35) (layer F.Cu) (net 15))
 (segment (start 143.955 92.075) (end 145.230001 93.350001) (width 0.35) (layer F.Cu) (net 15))
 (segment (start 148.9025 86.655) (end 150.297831 86.655) (width 0.35) (layer F.Cu) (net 8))
 (segment (start 150.297831 86.655) (end 151.765 88.122169) (width 0.35) (layer F.Cu) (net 8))
 (segment (start 151.765 88.122169) (end 151.765 90.17) (width 0.35) (layer F.Cu) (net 8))
 (segment (start 151.765 90.17) (end 153.67 92.075) (width 0.35) (layer F.Cu) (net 8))
 (segment (start 148.9025 87.305) (end 150.17 87.305) (width 0.35) (layer F.Cu) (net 7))
 (segment (start 150.17 87.305) (end 151.13 88.265) (width 0.35) (layer F.Cu) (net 7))
 (segment (start 151.13 88.265) (end 151.13 92.075) (width 0.35) (layer F.Cu) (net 7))
 (segment (start 156.169 89.255) (end 156.464 89.55) (width 0.35) (layer F.Cu) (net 16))
 (segment (start 154.6275 89.255) (end 156.169 89.255) (width 0.35) (layer F.Cu) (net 16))
 (via (at 152.4 84.455) (size 0.8) (drill 0.4) (layers F.Cu B.Cu) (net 5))
 (segment (start 153.3 85.355) (end 152.4 84.455) (width 0.35) (layer F.Cu) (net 5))
 (segment (start 154.6275 85.355) (end 153.3 85.355) (width 0.35) (layer F.Cu) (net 5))
 (segment (start 152.000001 84.055001) (end 152.4 84.455) (width 0.35) (layer B.Cu) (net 5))
 (segment (start 144.859997 84.055001) (end 152.000001 84.055001) (width 0.35) (layer B.Cu) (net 5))
 (segment (start 144.145 84.769998) (end 144.859997 84.055001) (width 0.35) (layer B.Cu) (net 5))
 (segment (start 140.48501 86.604999) (end 140.324999 86.76501) (width 0.35) (layer B.Cu) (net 5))
 (segment (start 143.060003 86.604999) (end 140.48501 86.604999) (width 0.35) (layer B.Cu) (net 5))
 (segment (start 144.145 85.520002) (end 143.060003 86.604999) (width 0.35) (layer B.Cu) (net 5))
 (segment (start 144.145 84.769998) (end 144.145 85.520002) (width 0.35) (layer B.Cu) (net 5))
 (segment (start 140.324999 86.76501) (end 140.324999 88.889999) (width 0.35) (layer B.Cu) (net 5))
 (segment (start 141.345 89.91) (end 141.85 89.91) (width 0.35) (layer B.Cu) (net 5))
 (segment (start 140.324999 88.889999) (end 141.345 89.91) (width 0.35) (layer B.Cu) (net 5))
 (segment (start 136.525 92.71) (end 155.575 92.71) (width 2.5) (layer B.Cu) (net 22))
 (segment (start 138.875 90.805) (end 140.145 92.075) (width 0.35) (layer F.Cu) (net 21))
 (segment (start 135.89 90.805) (end 138.875 90.805) (width 0.35) (layer F.Cu) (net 21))
 (segment (start 155.575 85.09) (end 154.94 85.09) (width 2.5) (layer B.Cu) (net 6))
 (segment (start 149.424999 86.355001) (end 148.15 87.63) (width 2.5) (layer B.Cu) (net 6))
 (segment (start 153.674999 86.355001) (end 149.424999 86.355001) (width 2.5) (layer B.Cu) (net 6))
 (segment (start 154.94 85.09) (end 153.674999 86.355001) (width 2.5) (layer B.Cu) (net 6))
 (segment (start 141.85 87.63) (end 148.15 87.63) (width 1.2) (layer B.Cu) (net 6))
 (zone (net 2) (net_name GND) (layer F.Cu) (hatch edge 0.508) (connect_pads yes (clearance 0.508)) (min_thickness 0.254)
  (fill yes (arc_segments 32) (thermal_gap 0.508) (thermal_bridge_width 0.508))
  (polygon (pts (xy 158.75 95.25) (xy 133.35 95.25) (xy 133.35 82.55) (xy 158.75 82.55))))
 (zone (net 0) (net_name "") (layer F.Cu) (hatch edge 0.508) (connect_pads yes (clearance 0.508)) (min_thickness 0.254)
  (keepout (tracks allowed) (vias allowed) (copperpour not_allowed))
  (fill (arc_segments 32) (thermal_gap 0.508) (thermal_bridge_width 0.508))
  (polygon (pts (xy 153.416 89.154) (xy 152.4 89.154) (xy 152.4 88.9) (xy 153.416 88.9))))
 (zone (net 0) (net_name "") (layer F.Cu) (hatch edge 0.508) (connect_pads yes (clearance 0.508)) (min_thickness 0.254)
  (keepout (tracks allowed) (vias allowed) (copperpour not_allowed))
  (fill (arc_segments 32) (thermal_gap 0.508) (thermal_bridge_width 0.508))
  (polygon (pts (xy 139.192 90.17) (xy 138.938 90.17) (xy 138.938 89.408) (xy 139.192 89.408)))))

